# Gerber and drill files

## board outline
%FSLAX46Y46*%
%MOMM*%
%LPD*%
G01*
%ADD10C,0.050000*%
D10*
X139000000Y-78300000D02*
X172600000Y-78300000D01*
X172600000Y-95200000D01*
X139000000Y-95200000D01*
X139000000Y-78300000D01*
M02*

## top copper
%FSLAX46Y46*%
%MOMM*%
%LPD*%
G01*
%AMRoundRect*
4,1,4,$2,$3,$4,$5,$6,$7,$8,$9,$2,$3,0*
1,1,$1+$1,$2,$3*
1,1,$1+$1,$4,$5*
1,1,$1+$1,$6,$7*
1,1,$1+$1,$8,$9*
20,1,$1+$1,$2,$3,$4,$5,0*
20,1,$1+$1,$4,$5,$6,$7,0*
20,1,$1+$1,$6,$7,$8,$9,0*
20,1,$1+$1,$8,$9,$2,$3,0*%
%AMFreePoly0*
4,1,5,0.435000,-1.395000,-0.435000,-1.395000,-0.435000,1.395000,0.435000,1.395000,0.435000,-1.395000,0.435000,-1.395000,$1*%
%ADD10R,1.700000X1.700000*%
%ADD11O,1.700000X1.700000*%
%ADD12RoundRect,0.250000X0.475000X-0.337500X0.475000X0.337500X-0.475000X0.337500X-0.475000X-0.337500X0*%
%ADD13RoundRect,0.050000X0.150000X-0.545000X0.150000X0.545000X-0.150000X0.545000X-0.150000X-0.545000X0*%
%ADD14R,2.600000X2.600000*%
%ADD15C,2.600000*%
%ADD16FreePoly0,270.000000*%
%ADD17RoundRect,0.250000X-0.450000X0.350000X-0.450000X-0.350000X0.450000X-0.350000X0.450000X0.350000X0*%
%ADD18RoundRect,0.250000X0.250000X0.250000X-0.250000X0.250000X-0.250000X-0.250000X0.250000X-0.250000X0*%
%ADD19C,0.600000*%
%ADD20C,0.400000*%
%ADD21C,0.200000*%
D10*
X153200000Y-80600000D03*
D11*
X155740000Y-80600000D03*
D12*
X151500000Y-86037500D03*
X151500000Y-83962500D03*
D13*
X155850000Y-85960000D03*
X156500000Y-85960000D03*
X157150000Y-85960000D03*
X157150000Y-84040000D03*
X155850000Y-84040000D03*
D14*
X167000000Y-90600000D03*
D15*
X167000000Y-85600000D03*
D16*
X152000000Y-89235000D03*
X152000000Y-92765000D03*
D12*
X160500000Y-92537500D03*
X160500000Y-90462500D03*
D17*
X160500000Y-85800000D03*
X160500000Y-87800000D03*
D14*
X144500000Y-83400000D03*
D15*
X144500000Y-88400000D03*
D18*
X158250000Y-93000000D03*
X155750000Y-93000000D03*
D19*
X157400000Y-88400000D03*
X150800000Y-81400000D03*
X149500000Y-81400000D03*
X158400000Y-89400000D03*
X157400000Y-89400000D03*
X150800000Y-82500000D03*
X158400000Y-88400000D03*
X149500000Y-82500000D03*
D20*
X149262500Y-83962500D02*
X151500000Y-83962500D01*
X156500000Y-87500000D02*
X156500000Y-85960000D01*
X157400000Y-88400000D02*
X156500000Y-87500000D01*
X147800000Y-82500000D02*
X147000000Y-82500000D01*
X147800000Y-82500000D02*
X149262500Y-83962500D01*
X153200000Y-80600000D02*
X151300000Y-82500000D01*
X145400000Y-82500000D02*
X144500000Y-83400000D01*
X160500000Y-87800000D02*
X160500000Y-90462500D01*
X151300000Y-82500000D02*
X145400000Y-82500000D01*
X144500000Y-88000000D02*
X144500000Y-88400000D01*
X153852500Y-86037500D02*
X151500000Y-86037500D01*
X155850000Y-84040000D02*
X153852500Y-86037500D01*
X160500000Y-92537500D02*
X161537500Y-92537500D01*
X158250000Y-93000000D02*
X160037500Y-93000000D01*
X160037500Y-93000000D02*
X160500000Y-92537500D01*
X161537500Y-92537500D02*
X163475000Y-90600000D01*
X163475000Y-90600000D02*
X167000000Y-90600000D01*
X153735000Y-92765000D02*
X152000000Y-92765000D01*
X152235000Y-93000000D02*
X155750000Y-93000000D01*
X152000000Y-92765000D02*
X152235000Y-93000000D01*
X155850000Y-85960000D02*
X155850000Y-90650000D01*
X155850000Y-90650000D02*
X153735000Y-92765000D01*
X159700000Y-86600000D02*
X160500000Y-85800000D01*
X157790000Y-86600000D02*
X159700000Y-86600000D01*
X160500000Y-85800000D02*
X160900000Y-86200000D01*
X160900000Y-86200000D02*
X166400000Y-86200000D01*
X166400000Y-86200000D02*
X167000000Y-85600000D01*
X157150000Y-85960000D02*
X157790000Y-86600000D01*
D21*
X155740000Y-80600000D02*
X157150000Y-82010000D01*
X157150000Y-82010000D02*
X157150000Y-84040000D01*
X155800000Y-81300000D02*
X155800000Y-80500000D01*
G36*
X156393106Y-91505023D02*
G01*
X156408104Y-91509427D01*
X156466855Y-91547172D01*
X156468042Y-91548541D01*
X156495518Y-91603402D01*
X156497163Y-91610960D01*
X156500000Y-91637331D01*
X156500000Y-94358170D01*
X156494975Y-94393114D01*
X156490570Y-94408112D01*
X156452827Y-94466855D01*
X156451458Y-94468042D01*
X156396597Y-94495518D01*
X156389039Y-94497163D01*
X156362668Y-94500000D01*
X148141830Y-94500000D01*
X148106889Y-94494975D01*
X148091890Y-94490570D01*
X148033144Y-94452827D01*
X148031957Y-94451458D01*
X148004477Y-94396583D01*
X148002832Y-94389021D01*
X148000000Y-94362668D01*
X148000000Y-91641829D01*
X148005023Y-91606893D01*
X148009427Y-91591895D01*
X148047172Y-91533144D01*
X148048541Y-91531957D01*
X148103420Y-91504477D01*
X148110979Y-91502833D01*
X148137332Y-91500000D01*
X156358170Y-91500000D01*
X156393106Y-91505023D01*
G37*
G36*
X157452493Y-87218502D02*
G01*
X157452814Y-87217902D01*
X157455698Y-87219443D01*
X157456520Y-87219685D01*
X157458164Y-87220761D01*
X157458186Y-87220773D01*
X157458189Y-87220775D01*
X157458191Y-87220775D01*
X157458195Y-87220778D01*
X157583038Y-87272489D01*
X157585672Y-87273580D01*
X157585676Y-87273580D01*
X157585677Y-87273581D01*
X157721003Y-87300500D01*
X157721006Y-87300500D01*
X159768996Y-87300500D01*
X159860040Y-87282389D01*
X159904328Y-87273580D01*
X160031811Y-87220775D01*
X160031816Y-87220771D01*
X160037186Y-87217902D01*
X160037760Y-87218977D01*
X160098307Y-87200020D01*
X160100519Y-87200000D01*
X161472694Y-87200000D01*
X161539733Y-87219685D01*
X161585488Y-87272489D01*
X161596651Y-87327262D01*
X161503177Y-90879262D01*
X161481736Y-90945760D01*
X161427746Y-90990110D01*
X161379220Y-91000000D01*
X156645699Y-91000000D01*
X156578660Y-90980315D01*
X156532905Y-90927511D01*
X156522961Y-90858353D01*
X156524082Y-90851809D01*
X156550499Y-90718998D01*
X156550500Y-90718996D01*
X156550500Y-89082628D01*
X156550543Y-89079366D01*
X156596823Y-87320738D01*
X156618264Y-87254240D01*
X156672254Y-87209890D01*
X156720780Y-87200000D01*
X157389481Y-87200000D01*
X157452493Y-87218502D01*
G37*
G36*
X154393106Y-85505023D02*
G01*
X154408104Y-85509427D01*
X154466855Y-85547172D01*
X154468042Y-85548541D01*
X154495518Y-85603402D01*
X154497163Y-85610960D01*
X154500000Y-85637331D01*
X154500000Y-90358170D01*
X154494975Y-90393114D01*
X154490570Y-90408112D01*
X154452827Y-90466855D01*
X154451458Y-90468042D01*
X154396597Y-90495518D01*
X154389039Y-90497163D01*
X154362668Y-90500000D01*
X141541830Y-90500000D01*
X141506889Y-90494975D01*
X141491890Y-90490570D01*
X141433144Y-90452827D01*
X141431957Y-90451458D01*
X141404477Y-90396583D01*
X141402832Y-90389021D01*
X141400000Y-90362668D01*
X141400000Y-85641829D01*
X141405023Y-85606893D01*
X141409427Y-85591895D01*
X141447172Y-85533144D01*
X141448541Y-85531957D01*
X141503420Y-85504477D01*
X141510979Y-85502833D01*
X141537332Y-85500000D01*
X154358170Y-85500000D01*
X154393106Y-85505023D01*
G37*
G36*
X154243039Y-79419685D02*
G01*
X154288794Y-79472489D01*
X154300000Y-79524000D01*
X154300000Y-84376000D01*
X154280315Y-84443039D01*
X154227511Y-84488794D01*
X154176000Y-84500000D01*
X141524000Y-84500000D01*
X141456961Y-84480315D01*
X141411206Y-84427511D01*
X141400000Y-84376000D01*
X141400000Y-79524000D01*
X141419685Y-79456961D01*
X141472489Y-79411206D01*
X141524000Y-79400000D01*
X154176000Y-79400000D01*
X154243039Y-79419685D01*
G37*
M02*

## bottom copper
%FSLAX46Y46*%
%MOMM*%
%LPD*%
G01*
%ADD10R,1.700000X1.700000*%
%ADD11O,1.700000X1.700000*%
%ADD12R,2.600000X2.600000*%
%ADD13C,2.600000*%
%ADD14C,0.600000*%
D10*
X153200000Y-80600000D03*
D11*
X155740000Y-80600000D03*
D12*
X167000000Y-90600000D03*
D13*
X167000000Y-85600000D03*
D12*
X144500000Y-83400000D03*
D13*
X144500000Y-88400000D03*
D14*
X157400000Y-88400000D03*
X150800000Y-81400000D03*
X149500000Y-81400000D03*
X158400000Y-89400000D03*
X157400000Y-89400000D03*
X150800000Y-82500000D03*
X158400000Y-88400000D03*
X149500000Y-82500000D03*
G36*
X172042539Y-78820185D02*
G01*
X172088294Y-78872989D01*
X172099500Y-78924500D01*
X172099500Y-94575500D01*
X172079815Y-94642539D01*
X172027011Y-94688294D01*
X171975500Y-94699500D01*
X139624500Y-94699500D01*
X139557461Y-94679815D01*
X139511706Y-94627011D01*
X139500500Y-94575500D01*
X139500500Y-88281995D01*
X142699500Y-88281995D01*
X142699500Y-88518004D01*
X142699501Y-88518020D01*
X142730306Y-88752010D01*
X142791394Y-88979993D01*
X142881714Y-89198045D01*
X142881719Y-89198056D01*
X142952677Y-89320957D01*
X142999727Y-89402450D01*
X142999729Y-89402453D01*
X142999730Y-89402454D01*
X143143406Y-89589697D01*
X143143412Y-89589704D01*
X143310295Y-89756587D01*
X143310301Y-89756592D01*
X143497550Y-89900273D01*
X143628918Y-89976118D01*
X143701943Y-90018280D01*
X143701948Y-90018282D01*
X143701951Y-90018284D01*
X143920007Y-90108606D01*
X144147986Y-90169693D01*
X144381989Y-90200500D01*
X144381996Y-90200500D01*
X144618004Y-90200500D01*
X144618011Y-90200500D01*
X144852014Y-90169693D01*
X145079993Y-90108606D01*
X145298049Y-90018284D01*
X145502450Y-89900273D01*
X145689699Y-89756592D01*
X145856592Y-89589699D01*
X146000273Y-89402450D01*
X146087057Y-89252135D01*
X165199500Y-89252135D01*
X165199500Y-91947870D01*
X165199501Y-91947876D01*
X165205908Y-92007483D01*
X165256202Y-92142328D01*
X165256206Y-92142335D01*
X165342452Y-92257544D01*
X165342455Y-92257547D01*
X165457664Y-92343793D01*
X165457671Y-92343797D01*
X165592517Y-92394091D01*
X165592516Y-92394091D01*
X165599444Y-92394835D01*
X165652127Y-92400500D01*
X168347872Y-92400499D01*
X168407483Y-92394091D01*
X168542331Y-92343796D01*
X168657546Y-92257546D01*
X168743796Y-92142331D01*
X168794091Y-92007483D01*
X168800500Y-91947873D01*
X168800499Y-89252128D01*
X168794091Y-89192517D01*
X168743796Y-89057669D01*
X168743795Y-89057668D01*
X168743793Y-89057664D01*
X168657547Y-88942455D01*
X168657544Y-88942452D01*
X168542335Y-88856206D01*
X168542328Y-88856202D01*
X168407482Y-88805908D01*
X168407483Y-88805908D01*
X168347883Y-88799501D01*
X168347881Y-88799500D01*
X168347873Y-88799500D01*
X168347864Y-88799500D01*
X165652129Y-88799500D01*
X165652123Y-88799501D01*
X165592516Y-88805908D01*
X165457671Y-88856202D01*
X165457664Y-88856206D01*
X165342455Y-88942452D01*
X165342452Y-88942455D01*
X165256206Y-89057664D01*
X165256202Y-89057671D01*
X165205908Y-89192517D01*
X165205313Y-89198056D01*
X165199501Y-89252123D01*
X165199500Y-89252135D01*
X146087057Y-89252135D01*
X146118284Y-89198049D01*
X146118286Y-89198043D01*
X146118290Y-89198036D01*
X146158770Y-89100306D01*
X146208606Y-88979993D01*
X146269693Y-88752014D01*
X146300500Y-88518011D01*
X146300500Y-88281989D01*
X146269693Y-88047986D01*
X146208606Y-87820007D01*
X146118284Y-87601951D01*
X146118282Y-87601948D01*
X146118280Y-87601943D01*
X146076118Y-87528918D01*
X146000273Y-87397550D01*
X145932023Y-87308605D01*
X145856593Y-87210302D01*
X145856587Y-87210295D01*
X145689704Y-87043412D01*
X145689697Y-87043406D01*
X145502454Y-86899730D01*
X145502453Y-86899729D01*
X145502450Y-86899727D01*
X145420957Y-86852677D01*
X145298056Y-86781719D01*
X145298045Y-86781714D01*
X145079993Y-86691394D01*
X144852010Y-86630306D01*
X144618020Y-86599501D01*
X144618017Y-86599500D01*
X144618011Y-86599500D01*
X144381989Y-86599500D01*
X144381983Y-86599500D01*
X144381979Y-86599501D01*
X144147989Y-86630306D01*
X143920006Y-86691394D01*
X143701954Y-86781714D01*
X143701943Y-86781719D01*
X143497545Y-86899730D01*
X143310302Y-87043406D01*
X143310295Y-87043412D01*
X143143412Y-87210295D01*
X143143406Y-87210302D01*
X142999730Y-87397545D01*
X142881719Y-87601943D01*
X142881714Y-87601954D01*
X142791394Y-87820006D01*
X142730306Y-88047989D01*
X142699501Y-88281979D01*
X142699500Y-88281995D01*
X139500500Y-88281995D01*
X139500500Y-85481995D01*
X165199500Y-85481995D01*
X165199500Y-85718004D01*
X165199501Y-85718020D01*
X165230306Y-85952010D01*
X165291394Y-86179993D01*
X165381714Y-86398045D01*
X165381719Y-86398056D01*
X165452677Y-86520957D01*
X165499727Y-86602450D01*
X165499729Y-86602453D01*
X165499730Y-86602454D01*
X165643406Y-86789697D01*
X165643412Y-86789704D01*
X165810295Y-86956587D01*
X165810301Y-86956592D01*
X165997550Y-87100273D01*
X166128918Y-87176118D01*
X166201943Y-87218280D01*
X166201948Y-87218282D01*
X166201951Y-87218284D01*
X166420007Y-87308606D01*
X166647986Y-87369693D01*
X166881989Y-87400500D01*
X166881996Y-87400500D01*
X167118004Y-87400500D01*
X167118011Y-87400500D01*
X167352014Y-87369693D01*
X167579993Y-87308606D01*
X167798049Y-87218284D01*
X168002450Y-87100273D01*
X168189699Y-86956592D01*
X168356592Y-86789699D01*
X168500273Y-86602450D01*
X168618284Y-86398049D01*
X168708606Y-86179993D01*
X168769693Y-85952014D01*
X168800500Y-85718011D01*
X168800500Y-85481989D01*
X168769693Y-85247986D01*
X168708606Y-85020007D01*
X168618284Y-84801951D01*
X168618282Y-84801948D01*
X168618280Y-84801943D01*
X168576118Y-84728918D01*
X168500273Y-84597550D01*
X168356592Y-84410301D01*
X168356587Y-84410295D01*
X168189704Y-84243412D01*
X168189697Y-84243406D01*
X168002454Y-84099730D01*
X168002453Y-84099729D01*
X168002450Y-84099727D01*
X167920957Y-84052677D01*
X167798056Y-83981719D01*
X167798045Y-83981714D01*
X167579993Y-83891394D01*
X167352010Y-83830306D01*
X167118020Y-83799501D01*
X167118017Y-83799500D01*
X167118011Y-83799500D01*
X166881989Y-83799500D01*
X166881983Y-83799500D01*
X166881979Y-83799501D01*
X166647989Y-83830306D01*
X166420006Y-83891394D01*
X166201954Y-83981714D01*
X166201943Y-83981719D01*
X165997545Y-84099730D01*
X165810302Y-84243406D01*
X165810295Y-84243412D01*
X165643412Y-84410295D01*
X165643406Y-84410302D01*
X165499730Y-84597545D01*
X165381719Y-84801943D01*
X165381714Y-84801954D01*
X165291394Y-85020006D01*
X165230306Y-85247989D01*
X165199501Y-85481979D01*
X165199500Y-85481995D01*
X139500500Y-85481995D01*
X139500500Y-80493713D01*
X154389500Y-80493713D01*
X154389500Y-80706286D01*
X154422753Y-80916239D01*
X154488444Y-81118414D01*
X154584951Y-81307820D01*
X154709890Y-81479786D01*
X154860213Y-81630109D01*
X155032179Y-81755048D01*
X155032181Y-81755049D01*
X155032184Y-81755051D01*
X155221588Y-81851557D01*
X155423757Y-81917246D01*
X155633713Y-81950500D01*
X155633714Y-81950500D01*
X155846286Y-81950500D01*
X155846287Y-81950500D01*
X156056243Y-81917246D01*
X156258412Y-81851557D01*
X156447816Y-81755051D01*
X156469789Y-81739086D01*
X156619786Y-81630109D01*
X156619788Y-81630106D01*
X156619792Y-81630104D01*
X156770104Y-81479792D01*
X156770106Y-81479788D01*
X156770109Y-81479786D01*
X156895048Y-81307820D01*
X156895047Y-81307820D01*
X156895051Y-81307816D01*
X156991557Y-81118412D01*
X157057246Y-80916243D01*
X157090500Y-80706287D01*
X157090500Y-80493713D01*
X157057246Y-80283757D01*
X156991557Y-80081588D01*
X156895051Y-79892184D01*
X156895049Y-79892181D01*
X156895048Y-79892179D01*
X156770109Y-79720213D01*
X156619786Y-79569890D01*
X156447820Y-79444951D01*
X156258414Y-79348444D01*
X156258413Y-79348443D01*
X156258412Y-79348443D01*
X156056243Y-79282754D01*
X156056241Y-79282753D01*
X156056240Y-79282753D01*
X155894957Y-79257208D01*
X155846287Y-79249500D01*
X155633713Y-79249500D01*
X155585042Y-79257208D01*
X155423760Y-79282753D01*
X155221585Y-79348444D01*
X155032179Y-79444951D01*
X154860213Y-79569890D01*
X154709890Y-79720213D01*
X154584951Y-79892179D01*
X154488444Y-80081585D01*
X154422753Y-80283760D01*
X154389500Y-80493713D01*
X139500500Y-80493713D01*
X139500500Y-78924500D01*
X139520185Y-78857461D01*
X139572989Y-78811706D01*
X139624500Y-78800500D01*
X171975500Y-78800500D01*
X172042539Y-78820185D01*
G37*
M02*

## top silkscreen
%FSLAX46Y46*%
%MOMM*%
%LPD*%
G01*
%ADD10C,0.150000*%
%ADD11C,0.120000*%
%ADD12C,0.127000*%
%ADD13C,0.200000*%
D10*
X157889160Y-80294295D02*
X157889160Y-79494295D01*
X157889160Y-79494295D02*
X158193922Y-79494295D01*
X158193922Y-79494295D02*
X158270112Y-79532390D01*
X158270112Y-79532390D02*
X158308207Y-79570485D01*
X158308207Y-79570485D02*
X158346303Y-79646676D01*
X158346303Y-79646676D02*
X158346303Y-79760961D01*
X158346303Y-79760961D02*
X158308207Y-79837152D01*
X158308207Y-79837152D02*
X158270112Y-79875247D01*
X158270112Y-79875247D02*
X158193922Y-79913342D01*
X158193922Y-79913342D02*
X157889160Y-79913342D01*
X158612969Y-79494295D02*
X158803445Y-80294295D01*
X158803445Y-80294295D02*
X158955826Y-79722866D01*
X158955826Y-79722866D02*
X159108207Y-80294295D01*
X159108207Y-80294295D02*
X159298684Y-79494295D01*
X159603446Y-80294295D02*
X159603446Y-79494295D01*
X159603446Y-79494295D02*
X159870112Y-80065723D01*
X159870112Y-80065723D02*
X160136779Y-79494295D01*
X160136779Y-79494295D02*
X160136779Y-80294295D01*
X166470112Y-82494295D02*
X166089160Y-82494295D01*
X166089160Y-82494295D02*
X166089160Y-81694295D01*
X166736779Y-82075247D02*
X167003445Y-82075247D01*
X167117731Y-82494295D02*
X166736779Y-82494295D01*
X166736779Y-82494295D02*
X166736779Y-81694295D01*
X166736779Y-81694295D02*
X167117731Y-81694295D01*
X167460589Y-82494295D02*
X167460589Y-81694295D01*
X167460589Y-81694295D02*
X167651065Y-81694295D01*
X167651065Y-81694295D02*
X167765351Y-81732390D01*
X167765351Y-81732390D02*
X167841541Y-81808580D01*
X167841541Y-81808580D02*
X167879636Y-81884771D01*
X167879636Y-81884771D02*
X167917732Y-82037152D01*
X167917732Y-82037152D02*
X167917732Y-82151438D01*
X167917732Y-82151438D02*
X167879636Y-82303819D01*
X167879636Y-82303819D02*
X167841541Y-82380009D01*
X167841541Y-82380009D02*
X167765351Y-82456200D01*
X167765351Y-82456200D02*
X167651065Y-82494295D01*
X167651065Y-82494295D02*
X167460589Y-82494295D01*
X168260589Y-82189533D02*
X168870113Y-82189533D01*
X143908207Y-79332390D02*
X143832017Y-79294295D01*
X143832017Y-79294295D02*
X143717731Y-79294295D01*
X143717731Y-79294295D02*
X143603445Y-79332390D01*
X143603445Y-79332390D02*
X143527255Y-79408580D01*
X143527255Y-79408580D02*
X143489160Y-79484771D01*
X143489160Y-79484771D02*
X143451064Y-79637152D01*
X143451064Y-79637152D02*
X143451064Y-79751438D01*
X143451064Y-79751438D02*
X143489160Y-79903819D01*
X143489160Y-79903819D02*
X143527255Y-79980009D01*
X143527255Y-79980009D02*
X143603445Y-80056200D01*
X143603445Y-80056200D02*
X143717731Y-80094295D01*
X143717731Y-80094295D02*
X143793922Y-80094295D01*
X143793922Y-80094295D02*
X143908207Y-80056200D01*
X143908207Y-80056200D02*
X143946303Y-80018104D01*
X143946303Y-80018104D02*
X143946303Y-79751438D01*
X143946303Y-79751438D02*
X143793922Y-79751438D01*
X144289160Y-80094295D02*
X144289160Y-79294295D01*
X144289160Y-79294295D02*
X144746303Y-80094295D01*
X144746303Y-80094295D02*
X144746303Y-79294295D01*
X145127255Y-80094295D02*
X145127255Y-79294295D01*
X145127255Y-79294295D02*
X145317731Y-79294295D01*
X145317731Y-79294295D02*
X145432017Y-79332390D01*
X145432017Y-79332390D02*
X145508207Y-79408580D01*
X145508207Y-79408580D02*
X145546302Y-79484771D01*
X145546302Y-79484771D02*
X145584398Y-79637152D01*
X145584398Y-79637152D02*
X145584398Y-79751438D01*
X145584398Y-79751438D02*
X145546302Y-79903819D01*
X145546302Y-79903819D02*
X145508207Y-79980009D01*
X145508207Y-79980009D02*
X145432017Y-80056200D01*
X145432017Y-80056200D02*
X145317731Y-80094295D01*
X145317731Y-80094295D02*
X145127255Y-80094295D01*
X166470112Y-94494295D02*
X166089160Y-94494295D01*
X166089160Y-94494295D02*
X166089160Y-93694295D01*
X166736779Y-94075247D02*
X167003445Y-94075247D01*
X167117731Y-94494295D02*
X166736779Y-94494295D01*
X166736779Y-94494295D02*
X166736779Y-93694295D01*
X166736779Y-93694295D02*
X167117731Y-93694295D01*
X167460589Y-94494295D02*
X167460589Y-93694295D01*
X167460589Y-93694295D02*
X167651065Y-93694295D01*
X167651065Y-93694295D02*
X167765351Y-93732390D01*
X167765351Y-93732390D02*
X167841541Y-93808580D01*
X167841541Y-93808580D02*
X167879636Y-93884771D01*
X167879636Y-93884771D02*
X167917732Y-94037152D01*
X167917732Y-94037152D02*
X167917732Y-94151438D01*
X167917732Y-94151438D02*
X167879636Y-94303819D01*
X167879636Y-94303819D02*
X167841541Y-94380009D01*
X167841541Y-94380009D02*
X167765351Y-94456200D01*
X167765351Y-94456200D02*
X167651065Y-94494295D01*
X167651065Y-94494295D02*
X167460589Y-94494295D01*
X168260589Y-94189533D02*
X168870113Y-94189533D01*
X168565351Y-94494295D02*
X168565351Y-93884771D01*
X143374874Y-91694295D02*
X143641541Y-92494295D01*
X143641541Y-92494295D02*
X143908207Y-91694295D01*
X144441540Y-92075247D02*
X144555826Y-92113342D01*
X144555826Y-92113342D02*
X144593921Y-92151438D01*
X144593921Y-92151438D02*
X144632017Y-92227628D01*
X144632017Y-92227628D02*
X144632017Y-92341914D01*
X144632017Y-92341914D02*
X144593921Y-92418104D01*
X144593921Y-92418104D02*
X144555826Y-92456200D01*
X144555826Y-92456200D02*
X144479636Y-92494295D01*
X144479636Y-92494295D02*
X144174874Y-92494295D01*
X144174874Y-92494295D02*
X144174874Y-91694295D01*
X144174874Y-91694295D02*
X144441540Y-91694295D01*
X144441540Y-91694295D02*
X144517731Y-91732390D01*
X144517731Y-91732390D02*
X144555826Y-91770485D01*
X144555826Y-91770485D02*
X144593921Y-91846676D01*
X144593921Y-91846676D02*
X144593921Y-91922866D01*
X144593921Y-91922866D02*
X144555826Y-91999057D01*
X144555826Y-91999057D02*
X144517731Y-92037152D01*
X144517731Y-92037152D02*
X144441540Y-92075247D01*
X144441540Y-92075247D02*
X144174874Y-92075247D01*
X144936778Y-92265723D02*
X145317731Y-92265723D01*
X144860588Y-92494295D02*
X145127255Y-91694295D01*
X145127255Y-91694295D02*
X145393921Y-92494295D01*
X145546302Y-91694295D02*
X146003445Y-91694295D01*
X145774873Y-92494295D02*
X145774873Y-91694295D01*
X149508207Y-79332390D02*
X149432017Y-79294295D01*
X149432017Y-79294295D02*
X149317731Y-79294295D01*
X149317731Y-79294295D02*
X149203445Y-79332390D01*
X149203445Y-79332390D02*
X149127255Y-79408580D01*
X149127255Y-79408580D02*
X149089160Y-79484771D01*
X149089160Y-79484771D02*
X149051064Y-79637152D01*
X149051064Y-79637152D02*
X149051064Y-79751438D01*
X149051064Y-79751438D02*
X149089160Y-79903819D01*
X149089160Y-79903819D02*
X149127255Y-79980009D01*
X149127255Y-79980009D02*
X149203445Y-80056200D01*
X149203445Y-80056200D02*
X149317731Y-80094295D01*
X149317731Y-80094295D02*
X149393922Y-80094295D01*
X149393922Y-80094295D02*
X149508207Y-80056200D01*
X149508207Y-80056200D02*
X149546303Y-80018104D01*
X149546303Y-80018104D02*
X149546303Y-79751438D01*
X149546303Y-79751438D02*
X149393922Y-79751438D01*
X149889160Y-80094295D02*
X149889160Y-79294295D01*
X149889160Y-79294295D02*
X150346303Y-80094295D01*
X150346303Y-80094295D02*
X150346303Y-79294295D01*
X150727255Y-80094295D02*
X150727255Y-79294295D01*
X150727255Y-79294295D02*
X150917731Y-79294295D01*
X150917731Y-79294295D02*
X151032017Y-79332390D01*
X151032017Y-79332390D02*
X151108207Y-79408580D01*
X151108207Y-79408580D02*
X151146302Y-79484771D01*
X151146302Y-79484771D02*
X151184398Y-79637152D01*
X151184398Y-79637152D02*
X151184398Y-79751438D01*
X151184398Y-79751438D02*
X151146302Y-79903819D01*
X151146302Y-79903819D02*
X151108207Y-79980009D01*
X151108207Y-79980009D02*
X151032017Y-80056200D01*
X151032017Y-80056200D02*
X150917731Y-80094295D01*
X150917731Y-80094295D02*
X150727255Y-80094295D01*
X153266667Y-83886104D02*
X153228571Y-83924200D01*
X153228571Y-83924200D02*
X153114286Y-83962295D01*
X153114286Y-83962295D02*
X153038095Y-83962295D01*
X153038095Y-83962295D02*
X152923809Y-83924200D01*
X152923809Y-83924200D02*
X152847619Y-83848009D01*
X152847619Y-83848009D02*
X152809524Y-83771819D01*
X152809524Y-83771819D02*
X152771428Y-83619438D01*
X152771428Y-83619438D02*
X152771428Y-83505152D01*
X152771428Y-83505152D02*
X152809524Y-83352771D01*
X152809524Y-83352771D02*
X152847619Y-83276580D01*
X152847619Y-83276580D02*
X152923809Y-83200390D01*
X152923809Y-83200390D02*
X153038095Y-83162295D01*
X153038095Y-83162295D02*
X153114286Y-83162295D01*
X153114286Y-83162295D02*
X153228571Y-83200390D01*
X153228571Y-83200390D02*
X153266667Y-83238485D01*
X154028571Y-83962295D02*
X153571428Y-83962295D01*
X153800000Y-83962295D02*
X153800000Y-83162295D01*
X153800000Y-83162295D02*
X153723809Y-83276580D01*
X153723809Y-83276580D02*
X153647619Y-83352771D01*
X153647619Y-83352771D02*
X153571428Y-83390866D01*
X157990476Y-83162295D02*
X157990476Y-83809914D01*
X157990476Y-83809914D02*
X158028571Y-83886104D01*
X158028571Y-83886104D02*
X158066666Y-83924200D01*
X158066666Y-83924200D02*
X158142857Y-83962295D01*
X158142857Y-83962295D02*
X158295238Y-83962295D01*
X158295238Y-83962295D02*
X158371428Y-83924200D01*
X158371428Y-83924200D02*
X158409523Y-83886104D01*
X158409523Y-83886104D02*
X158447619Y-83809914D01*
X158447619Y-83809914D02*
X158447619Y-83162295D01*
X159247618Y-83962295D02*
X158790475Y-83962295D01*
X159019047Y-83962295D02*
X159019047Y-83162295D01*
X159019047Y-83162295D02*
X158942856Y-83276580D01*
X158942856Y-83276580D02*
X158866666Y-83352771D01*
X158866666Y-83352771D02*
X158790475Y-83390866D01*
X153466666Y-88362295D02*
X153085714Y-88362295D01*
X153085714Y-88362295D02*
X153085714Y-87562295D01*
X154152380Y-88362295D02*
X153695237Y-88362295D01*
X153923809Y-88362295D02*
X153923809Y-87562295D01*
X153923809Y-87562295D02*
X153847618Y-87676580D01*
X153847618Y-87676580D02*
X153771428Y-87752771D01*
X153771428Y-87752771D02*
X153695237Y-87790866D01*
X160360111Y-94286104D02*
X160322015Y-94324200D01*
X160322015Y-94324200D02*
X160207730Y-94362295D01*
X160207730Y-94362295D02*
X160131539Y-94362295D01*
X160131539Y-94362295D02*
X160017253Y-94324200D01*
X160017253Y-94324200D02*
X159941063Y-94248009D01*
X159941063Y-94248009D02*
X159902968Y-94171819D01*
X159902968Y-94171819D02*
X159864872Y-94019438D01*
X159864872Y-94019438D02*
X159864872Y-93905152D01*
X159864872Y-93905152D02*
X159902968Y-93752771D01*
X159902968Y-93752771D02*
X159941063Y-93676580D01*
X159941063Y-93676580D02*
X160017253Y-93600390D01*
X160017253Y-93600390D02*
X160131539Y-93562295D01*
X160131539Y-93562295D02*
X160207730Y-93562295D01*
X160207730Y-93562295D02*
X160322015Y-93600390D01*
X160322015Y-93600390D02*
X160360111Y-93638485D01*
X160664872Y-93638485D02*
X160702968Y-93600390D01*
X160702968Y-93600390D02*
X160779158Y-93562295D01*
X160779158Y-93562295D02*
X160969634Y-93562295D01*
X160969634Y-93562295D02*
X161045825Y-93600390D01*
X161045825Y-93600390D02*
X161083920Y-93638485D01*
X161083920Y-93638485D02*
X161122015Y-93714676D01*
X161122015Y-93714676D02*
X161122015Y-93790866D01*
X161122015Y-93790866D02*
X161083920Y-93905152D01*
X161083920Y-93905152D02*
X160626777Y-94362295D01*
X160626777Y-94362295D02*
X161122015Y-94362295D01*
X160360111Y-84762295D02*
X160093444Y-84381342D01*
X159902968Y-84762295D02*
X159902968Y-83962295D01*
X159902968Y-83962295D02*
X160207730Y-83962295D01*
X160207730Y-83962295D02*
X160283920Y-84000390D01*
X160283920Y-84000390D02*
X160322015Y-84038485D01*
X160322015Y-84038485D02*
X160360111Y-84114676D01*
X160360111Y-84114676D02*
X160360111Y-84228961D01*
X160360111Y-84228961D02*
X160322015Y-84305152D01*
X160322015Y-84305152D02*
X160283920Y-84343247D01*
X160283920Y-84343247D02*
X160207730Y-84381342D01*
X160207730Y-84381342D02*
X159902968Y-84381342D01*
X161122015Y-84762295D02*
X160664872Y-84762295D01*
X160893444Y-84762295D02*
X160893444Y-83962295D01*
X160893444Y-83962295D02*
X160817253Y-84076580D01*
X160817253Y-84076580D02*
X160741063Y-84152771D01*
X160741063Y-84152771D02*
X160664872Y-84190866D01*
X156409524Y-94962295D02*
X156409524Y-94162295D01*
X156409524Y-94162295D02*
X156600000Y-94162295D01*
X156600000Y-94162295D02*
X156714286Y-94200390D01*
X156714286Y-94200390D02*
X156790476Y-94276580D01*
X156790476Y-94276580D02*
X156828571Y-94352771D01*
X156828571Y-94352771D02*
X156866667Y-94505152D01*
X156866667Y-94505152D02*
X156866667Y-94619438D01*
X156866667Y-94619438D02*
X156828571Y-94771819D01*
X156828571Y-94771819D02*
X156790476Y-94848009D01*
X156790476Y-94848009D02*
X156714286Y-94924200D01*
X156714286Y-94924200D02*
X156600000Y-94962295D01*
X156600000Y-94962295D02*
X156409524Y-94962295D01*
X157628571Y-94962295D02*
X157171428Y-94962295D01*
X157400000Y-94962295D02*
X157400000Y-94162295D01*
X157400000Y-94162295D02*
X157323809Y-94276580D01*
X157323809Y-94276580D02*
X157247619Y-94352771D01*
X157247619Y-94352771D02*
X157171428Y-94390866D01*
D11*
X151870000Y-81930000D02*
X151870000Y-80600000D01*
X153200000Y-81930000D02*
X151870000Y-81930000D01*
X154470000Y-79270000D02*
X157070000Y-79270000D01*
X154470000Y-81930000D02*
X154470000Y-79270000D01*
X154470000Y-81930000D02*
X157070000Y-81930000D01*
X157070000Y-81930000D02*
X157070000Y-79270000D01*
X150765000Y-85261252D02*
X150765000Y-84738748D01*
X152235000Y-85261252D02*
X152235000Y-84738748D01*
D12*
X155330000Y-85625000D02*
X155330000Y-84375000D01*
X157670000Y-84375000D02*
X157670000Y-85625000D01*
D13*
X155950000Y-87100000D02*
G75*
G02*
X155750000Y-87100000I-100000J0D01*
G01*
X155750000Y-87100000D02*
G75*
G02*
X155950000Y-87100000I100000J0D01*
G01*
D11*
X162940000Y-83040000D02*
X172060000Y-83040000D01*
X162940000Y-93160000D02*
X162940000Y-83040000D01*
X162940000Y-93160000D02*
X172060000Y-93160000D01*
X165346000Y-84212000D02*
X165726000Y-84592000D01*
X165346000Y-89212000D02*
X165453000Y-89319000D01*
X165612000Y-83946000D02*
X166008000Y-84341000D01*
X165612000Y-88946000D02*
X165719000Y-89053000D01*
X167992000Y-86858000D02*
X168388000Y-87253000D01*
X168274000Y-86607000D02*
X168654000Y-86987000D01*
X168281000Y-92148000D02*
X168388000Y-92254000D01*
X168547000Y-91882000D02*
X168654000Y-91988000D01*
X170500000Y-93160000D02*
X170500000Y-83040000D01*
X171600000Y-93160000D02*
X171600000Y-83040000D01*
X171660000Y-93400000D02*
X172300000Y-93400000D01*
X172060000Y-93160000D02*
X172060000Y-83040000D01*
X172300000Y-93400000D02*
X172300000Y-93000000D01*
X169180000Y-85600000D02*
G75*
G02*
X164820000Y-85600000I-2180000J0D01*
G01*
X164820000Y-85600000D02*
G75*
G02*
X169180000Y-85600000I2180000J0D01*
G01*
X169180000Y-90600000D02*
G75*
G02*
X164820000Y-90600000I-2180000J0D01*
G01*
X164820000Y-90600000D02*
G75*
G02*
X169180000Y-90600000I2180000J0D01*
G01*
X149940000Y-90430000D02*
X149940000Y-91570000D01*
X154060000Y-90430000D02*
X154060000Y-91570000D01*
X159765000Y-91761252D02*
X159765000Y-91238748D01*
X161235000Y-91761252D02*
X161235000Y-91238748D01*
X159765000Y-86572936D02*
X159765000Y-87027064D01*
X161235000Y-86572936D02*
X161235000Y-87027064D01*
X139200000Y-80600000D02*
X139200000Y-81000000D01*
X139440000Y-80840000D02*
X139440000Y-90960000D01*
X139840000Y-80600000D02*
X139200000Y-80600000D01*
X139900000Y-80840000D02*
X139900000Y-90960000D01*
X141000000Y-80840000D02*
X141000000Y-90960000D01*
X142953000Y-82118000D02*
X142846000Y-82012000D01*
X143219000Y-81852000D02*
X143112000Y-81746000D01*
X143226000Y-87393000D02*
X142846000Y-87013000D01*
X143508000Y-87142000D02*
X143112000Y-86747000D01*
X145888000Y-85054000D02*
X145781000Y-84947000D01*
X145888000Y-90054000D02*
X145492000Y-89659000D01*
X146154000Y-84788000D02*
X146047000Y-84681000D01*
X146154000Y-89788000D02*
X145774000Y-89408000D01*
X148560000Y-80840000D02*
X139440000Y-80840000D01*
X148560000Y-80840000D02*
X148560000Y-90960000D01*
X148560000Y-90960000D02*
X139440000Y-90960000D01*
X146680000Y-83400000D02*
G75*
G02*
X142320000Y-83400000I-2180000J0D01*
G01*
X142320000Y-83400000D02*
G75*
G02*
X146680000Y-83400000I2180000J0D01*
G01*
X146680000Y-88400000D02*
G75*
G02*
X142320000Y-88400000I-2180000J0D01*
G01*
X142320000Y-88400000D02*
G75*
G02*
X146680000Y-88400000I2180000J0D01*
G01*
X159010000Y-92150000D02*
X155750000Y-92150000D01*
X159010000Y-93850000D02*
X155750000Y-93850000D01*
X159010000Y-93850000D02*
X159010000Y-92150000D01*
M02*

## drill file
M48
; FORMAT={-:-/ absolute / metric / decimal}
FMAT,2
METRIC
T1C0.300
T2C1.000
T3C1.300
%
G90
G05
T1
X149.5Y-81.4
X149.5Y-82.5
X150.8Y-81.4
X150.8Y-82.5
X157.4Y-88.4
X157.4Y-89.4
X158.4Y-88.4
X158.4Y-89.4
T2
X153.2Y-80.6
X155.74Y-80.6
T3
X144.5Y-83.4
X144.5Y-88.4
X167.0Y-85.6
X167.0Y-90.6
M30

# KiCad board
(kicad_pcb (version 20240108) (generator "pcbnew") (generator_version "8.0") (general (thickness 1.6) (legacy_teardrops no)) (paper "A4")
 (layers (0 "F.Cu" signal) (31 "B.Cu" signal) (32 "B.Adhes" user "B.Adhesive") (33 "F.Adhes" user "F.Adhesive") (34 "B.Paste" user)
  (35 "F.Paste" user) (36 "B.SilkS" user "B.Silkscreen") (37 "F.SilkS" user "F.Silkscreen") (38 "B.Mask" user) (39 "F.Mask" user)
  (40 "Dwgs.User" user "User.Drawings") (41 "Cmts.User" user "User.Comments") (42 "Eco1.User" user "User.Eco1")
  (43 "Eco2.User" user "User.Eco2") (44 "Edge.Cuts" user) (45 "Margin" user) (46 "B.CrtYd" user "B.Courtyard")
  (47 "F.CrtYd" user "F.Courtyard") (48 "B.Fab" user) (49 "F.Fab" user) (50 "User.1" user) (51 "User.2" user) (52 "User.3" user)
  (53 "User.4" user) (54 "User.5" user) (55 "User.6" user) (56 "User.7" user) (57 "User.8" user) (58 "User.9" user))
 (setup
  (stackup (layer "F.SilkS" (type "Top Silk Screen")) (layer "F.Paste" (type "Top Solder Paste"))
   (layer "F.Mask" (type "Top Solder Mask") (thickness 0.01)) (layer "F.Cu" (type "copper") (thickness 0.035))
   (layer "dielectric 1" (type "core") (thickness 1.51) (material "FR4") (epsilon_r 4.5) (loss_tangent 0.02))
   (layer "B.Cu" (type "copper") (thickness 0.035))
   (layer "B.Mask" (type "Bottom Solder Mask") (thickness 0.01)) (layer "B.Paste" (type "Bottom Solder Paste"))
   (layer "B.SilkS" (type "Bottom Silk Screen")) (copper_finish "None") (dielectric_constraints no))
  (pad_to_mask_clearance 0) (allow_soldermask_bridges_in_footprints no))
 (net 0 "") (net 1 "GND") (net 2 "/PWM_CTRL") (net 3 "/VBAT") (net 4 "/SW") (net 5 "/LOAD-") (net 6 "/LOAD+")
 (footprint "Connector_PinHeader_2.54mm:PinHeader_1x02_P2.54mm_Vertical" (layer "F.Cu") (at 153.2 80.6 90)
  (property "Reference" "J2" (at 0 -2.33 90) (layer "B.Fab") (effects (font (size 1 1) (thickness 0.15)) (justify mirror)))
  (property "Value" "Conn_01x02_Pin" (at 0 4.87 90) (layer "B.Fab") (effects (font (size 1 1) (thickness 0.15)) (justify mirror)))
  (fp_line (start -1.33 -1.33) (end 0 -1.33) (stroke (width 0.12) (type solid)) (layer "F.SilkS"))
  (fp_line (start -1.33 0) (end -1.33 -1.33) (stroke (width 0.12) (type solid)) (layer "F.SilkS"))
  (fp_line (start 1.33 1.27) (end 1.33 3.87) (stroke (width 0.12) (type solid)) (layer "F.SilkS"))
  (fp_line (start -1.33 1.27) (end 1.33 1.27) (stroke (width 0.12) (type solid)) (layer "F.SilkS"))
  (fp_line (start -1.33 1.27) (end -1.33 3.87) (stroke (width 0.12) (type solid)) (layer "F.SilkS"))
  (fp_line (start -1.33 3.87) (end 1.33 3.87) (stroke (width 0.12) (type solid)) (layer "F.SilkS"))
  (pad "1" thru_hole rect (at 0 0 90) (size 1.7 1.7) (drill 1) (layers "*.Cu" "*.Mask") (remove_unused_layers no) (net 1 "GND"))
  (pad "2" thru_hole oval (at 0 2.54 90) (size 1.7 1.7) (drill 1) (layers "*.Cu" "*.Mask") (remove_unused_layers no) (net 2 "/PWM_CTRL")))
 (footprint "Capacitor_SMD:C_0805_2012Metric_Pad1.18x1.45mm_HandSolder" (layer "F.Cu") (at 151.5 85 90)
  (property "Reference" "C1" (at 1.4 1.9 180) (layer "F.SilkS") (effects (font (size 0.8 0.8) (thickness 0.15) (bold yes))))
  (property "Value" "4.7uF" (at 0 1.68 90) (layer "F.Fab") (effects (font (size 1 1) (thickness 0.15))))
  (fp_line (start -0.261252 -0.735) (end 0.261252 -0.735) (stroke (width 0.12) (type solid)) (layer "F.SilkS"))
  (fp_line (start -0.261252 0.735) (end 0.261252 0.735) (stroke (width 0.12) (type solid)) (layer "F.SilkS"))
  (pad "1" smd roundrect (at -1.0375 0 90) (size 1.175 1.45) (layers "F.Cu" "F.Paste" "F.Mask") (roundrect_rratio 0.212766) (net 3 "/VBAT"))
  (pad "2" smd roundrect (at 1.0375 0 90) (size 1.175 1.45) (layers "F.Cu" "F.Paste" "F.Mask") (roundrect_rratio 0.212766) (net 1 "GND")))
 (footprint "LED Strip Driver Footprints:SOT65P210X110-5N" (layer "F.Cu") (at 156.5 85 90)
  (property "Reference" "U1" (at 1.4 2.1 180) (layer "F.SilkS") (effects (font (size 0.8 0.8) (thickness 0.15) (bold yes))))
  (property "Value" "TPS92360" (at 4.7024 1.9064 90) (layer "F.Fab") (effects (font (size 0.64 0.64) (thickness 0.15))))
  (fp_line (start -0.625 -1.17) (end 0.625 -1.17) (stroke (width 0.127) (type solid)) (layer "F.SilkS"))
  (fp_line (start 0.625 1.17) (end -0.625 1.17) (stroke (width 0.127) (type solid)) (layer "F.SilkS"))
  (fp_circle (center -2.1 -0.65) (end -2 -0.65) (stroke (width 0.2) (type solid)) (fill none) (layer "F.SilkS"))
  (pad "1" smd roundrect (at -0.96 -0.65 90) (size 1.19 0.4) (layers "F.Cu" "F.Paste" "F.Mask") (roundrect_rratio 0.125) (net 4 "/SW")
   (solder_mask_margin 0.102))
  (pad "2" smd roundrect (at -0.96 0 90) (size 1.19 0.4) (layers "F.Cu" "F.Paste" "F.Mask") (roundrect_rratio 0.125) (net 1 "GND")
   (solder_mask_margin 0.102))
  (pad "3" smd roundrect (at -0.96 0.65 90) (size 1.19 0.4) (layers "F.Cu" "F.Paste" "F.Mask") (roundrect_rratio 0.125) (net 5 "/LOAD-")
   (solder_mask_margin 0.102))
  (pad "4" smd roundrect (at 0.96 0.65 90) (size 1.19 0.4) (layers "F.Cu" "F.Paste" "F.Mask") (roundrect_rratio 0.125) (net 2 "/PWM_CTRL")
   (solder_mask_margin 0.102))
  (pad "5" smd roundrect (at 0.96 -0.65 90) (size 1.19 0.4) (layers "F.Cu" "F.Paste" "F.Mask") (roundrect_rratio 0.125) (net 3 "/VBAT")
   (solder_mask_margin 0.102)))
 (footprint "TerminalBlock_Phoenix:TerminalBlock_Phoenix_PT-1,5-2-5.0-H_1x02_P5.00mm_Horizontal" (layer "F.Cu") (at 167 90.6 90)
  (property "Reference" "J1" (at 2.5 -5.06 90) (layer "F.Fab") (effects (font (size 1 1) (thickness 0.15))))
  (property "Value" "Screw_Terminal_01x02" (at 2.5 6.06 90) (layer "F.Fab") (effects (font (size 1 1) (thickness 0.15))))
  (fp_line (start 7.56 -4.06) (end 7.56 5.06) (stroke (width 0.12) (type solid)) (layer "F.SilkS"))
  (fp_line (start -2.56 -4.06) (end 7.56 -4.06) (stroke (width 0.12) (type solid)) (layer "F.SilkS"))
  (fp_line (start -2.56 -4.06) (end -2.56 5.06) (stroke (width 0.12) (type solid)) (layer "F.SilkS"))
  (fp_line (start 6.388 -1.654) (end 6.008 -1.274) (stroke (width 0.12) (type solid)) (layer "F.SilkS"))
  (fp_line (start 1.388 -1.654) (end 1.281 -1.547) (stroke (width 0.12) (type solid)) (layer "F.SilkS"))
  (fp_line (start 6.654 -1.388) (end 6.259 -0.992) (stroke (width 0.12) (type solid)) (layer "F.SilkS"))
  (fp_line (start 1.654 -1.388) (end 1.547 -1.281) (stroke (width 0.12) (type solid)) (layer "F.SilkS"))
  (fp_line (start 3.742 0.992) (end 3.347 1.388) (stroke (width 0.12) (type solid)) (layer "F.SilkS"))
  (fp_line (start 3.993 1.274) (end 3.613 1.654) (stroke (width 0.12) (type solid)) (layer "F.SilkS"))
  (fp_line (start -1.548 1.281) (end -1.654 1.388) (stroke (width 0.12) (type solid)) (layer "F.SilkS"))
  (fp_line (start -1.282 1.547) (end -1.388 1.654) (stroke (width 0.12) (type solid)) (layer "F.SilkS"))
  (fp_line (start -2.56 3.5) (end 7.56 3.5) (stroke (width 0.12) (type solid)) (layer "F.SilkS"))
  (fp_line (start -2.56 4.6) (end 7.56 4.6) (stroke (width 0.12) (type solid)) (layer "F.SilkS"))
  (fp_line (start -2.8 4.66) (end -2.8 5.3) (stroke (width 0.12) (type solid)) (layer "F.SilkS"))
  (fp_line (start -2.56 5.06) (end 7.56 5.06) (stroke (width 0.12) (type solid)) (layer "F.SilkS"))
  (fp_line (start -2.8 5.3) (end -2.4 5.3) (stroke (width 0.12) (type solid)) (layer "F.SilkS"))
  (fp_circle (center 5 0) (end 7.18 0) (stroke (width 0.12) (type solid)) (fill none) (layer "F.SilkS"))
  (fp_circle (center 0 0) (end 2.18 0) (stroke (width 0.12) (type solid)) (fill none) (layer "F.SilkS"))
  (pad "1" thru_hole rect (at 0 0 90) (size 2.6 2.6) (drill 1.3) (layers "*.Cu" "*.Mask") (remove_unused_layers no) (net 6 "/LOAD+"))
  (pad "2" thru_hole circle (at 5 0 90) (size 2.6 2.6) (drill 1.3) (layers "*.Cu" "*.Mask") (remove_unused_layers no) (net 5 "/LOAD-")))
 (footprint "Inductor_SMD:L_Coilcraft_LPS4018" (layer "F.Cu") (at 152 91 -90)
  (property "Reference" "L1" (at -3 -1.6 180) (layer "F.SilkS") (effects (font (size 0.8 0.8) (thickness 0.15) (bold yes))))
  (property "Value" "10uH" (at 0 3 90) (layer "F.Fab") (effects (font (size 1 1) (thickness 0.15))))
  (fp_line (start -0.57 2.06) (end 0.57 2.06) (stroke (width 0.12) (type solid)) (layer "F.SilkS"))
  (fp_line (start -0.57 -2.06) (end 0.57 -2.06) (stroke (width 0.12) (type solid)) (layer "F.SilkS"))
  (pad "1" smd custom (at -1.765 0 270) (size 0.87 2.79) (layers "F.Cu" "F.Paste" "F.Mask") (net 3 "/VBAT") (zone_connect 2)
   (options (clearance outline) (anchor rect)) (primitives))
  (pad "2" smd custom (at 1.765 0 270) (size 0.87 2.79) (layers "F.Cu" "F.Paste" "F.Mask") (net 4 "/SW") (zone_connect 2)
   (options (clearance outline) (anchor rect)) (primitives)))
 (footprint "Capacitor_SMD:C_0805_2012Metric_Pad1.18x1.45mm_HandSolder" (layer "F.Cu") (at 160.5 91.5 90)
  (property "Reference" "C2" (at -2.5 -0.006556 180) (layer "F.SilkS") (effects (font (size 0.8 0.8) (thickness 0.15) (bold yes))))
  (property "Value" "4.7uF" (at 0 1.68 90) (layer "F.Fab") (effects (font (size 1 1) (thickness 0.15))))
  (fp_line (start -0.261252 -0.735) (end 0.261252 -0.735) (stroke (width 0.12) (type solid)) (layer "F.SilkS"))
  (fp_line (start -0.261252 0.735) (end 0.261252 0.735) (stroke (width 0.12) (type solid)) (layer "F.SilkS"))
  (pad "1" smd roundrect (at -1.0375 0 90) (size 1.175 1.45) (layers "F.Cu" "F.Paste" "F.Mask") (roundrect_rratio 0.212766) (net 6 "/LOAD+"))
  (pad "2" smd roundrect (at 1.0375 0 90) (size 1.175 1.45) (layers "F.Cu" "F.Paste" "F.Mask") (roundrect_rratio 0.212766) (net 1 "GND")))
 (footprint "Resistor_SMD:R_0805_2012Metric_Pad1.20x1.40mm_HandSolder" (layer "F.Cu") (at 160.5 86.8 -90)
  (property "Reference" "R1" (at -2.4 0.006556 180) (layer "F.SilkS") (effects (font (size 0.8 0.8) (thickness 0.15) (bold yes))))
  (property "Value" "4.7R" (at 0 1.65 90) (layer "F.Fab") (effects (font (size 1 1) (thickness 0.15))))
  (fp_line (start -0.227064 0.735) (end 0.227064 0.735) (stroke (width 0.12) (type solid)) (layer "F.SilkS"))
  (fp_line (start -0.227064 -0.735) (end 0.227064 -0.735) (stroke (width 0.12) (type solid)) (layer "F.SilkS"))
  (pad "1" smd roundrect (at -1 0 270) (size 1.2 1.4) (layers "F.Cu" "F.Paste" "F.Mask") (roundrect_rratio 0.208333) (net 5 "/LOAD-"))
  (pad "2" smd roundrect (at 1 0 270) (size 1.2 1.4) (layers "F.Cu" "F.Paste" "F.Mask") (roundrect_rratio 0.208333) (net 1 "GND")))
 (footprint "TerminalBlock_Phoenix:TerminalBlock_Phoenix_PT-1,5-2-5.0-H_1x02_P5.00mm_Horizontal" (layer "F.Cu") (at 144.5 83.4 -90)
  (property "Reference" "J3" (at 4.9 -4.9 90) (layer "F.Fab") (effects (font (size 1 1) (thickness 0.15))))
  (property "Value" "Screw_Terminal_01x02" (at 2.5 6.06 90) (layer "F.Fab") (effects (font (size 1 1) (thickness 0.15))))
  (fp_line (start -2.8 5.3) (end -2.4 5.3) (stroke (width 0.12) (type solid)) (layer "F.SilkS"))
  (fp_line (start -2.56 5.06) (end 7.56 5.06) (stroke (width 0.12) (type solid)) (layer "F.SilkS"))
  (fp_line (start -2.8 4.66) (end -2.8 5.3) (stroke (width 0.12) (type solid)) (layer "F.SilkS"))
  (fp_line (start -2.56 4.6) (end 7.56 4.6) (stroke (width 0.12) (type solid)) (layer "F.SilkS"))
  (fp_line (start -2.56 3.5) (end 7.56 3.5) (stroke (width 0.12) (type solid)) (layer "F.SilkS"))
  (fp_line (start -1.282 1.547) (end -1.388 1.654) (stroke (width 0.12) (type solid)) (layer "F.SilkS"))
  (fp_line (start -1.548 1.281) (end -1.654 1.388) (stroke (width 0.12) (type solid)) (layer "F.SilkS"))
  (fp_line (start 3.993 1.274) (end 3.613 1.654) (stroke (width 0.12) (type solid)) (layer "F.SilkS"))
  (fp_line (start 3.742 0.992) (end 3.347 1.388) (stroke (width 0.12) (type solid)) (layer "F.SilkS"))
  (fp_line (start 1.654 -1.388) (end 1.547 -1.281) (stroke (width 0.12) (type solid)) (layer "F.SilkS"))
  (fp_line (start 6.654 -1.388) (end 6.259 -0.992) (stroke (width 0.12) (type solid)) (layer "F.SilkS"))
  (fp_line (start 1.388 -1.654) (end 1.281 -1.547) (stroke (width 0.12) (type solid)) (layer "F.SilkS"))
  (fp_line (start 6.388 -1.654) (end 6.008 -1.274) (stroke (width 0.12) (type solid)) (layer "F.SilkS"))
  (fp_line (start -2.56 -4.06) (end -2.56 5.06) (stroke (width 0.12) (type solid)) (layer "F.SilkS"))
  (fp_line (start -2.56 -4.06) (end 7.56 -4.06) (stroke (width 0.12) (type solid)) (layer "F.SilkS"))
  (fp_line (start 7.56 -4.06) (end 7.56 5.06) (stroke (width 0.12) (type solid)) (layer "F.SilkS"))
  (fp_circle (center 0 0) (end 2.18 0) (stroke (width 0.12) (type solid)) (fill none) (layer "F.SilkS"))
  (fp_circle (center 5 0) (end 7.18 0) (stroke (width 0.12) (type solid)) (fill none) (layer "F.SilkS"))
  (pad "1" thru_hole rect (at 0 0 270) (size 2.6 2.6) (drill 1.3) (layers "*.Cu" "*.Mask") (remove_unused_layers no) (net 1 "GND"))
  (pad "2" thru_hole circle (at 5 0 270) (size 2.6 2.6) (drill 1.3) (layers "*.Cu" "*.Mask") (remove_unused_layers no) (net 3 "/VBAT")))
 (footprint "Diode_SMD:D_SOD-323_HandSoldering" (layer "F.Cu") (at 157 93 180)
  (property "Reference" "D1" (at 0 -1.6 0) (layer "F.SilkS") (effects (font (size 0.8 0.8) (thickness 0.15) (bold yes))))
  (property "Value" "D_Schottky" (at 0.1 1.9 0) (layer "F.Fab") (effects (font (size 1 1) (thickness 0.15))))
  (fp_line (start -2.01 0.85) (end 1.25 0.85) (stroke (width 0.12) (type solid)) (layer "F.SilkS"))
  (fp_line (start -2.01 -0.85) (end 1.25 -0.85) (stroke (width 0.12) (type solid)) (layer "F.SilkS"))
  (fp_line (start -2.01 -0.85) (end -2.01 0.85) (stroke (width 0.12) (type solid)) (layer "F.SilkS"))
  (pad "1" smd roundrect (at -1.25 0 180) (size 1 1) (layers "F.Cu" "F.Paste" "F.Mask") (roundrect_rratio 0.25) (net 6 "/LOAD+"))
  (pad "2" smd roundrect (at 1.25 0 180) (size 1 1) (layers "F.Cu" "F.Paste" "F.Mask") (roundrect_rratio 0.25) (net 4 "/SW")))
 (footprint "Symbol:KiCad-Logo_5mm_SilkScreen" (layer "B.Cu") (at 156.005698 85.517938 180)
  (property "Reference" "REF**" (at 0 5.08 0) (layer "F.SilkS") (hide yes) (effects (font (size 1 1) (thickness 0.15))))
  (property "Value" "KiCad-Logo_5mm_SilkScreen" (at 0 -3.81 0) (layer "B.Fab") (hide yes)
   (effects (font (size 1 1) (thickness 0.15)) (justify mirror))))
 (gr_rect (start 139 78.3) (end 172.6 95.2) (stroke (width 0.05) (type default)) (fill none) (layer "Edge.Cuts"))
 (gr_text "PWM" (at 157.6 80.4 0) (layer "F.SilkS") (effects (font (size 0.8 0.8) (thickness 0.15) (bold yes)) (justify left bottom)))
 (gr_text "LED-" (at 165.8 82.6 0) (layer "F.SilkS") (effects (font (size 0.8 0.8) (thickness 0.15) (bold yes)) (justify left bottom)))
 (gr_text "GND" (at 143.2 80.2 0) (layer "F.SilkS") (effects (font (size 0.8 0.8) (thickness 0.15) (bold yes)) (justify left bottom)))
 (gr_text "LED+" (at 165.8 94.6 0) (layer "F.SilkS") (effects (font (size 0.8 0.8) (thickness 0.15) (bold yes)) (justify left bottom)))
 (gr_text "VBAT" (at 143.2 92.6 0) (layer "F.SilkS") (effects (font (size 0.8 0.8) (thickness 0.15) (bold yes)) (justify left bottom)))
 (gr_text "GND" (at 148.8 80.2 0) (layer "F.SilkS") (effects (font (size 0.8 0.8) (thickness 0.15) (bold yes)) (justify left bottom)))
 (segment (start 149.2625 83.9625) (end 151.5 83.9625) (width 0.4) (layer "F.Cu") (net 1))
 (segment (start 156.5 87.5) (end 156.5 85.96) (width 0.4) (layer "F.Cu") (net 1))
 (segment (start 157.4 88.4) (end 156.5 87.5) (width 0.4) (layer "F.Cu") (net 1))
 (segment (start 147.8 82.5) (end 147 82.5) (width 0.4) (layer "F.Cu") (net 1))
 (segment (start 147.8 82.5) (end 149.2625 83.9625) (width 0.4) (layer "F.Cu") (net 1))
 (segment (start 153.2 80.6) (end 151.3 82.5) (width 0.4) (layer "F.Cu") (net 1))
 (segment (start 145.4 82.5) (end 144.5 83.4) (width 0.4) (layer "F.Cu") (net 1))
 (segment (start 160.5 87.8) (end 160.5 90.4625) (width 0.4) (layer "F.Cu") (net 1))
 (segment (start 151.3 82.5) (end 145.4 82.5) (width 0.4) (layer "F.Cu") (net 1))
 (via (at 157.4 88.4) (size 0.6) (drill 0.3) (layers "F.Cu" "B.Cu") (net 1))
 (via (at 150.8 81.4) (size 0.6) (drill 0.3) (layers "F.Cu" "B.Cu") (free yes) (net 1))
 (via (at 149.5 81.4) (size 0.6) (drill 0.3) (layers "F.Cu" "B.Cu") (free yes) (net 1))
 (via (at 158.4 89.4) (size 0.6) (drill 0.3) (layers "F.Cu" "B.Cu") (free yes) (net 1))
 (via (at 157.4 89.4) (size 0.6) (drill 0.3) (layers "F.Cu" "B.Cu") (free yes) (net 1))
 (via (at 150.8 82.5) (size 0.6) (drill 0.3) (layers "F.Cu" "B.Cu") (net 1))
 (via (at 158.4 88.4) (size 0.6) (drill 0.3) (layers "F.Cu" "B.Cu") (free yes) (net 1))
 (via (at 149.5 82.5) (size 0.6) (drill 0.3) (layers "F.Cu" "B.Cu") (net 1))
 (segment (start 144.5 88) (end 144.5 88.4) (width 0.4) (layer "F.Cu") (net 3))
 (segment (start 153.8525 86.0375) (end 151.5 86.0375) (width 0.4) (layer "F.Cu") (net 3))
 (segment (start 155.85 84.04) (end 153.8525 86.0375) (width 0.4) (layer "F.Cu") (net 3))
 (segment (start 160.5 92.5375) (end 161.5375 92.5375) (width 0.4) (layer "F.Cu") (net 6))
 (segment (start 158.25 93) (end 160.0375 93) (width 0.4) (layer "F.Cu") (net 6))
 (segment (start 160.0375 93) (end 160.5 92.5375) (width 0.4) (layer "F.Cu") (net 6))
 (segment (start 161.5375 92.5375) (end 163.475 90.6) (width 0.4) (layer "F.Cu") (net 6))
 (segment (start 163.475 90.6) (end 167 90.6) (width 0.4) (layer "F.Cu") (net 6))
 (segment (start 153.735 92.765) (end 152 92.765) (width 0.4) (layer "F.Cu") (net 4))
 (segment (start 152.235 93) (end 155.75 93) (width 0.4) (layer "F.Cu") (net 4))
 (segment (start 152 92.765) (end 152.235 93) (width 0.4) (layer "F.Cu") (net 4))
 (segment (start 155.85 85.96) (end 155.85 90.65) (width 0.4) (layer "F.Cu") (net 4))
 (segment (start 155.85 90.65) (end 153.735 92.765) (width 0.4) (layer "F.Cu") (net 4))
 (segment (start 159.7 86.6) (end 160.5 85.8) (width 0.4) (layer "F.Cu") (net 5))
 (segment (start 157.79 86.6) (end 159.7 86.6) (width 0.4) (layer "F.Cu") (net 5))
 (segment (start 160.5 85.8) (end 160.9 86.2) (width 0.4) (layer "F.Cu") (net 5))
 (segment (start 160.9 86.2) (end 166.4 86.2) (width 0.4) (layer "F.Cu") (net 5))
 (segment (start 166.4 86.2) (end 167 85.6) (width 0.4) (layer "F.Cu") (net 5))
 (segment (start 157.15 85.96) (end 157.79 86.6) (width 0.4) (layer "F.Cu") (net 5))
 (segment (start 155.74 80.6) (end 157.15 82.01) (width 0.2) (layer "F.Cu") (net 2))
 (segment (start 157.15 82.01) (end 157.15 84.04) (width 0.2) (layer "F.Cu") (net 2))
 (segment (start 155.8 81.3) (end 155.8 80.5) (width 0.2) (layer "F.Cu") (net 2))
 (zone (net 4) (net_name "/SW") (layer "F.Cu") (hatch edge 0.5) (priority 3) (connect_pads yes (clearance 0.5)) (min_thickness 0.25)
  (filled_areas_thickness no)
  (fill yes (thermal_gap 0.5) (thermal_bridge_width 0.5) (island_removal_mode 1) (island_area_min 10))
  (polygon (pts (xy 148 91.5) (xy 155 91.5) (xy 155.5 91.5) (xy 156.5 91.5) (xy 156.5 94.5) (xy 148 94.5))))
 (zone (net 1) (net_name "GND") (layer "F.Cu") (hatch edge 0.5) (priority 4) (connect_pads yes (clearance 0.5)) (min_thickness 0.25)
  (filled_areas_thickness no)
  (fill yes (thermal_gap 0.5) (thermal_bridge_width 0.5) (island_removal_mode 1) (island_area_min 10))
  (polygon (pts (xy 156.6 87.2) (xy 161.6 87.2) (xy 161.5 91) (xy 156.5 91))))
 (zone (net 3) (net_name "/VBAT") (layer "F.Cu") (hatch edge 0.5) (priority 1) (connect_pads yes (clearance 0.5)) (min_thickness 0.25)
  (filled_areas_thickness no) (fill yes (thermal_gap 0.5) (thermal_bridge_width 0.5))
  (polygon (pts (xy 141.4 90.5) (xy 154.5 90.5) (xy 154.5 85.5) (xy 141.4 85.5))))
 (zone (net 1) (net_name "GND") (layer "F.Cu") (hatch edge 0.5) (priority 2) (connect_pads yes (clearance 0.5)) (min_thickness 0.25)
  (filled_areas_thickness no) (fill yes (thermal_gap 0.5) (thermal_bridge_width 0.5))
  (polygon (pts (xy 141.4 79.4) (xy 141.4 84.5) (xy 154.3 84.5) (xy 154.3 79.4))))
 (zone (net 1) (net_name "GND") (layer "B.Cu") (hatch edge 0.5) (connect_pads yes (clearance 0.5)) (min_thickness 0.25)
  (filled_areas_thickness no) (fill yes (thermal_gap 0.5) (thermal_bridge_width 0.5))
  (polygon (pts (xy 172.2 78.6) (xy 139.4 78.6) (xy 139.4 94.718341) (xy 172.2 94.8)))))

